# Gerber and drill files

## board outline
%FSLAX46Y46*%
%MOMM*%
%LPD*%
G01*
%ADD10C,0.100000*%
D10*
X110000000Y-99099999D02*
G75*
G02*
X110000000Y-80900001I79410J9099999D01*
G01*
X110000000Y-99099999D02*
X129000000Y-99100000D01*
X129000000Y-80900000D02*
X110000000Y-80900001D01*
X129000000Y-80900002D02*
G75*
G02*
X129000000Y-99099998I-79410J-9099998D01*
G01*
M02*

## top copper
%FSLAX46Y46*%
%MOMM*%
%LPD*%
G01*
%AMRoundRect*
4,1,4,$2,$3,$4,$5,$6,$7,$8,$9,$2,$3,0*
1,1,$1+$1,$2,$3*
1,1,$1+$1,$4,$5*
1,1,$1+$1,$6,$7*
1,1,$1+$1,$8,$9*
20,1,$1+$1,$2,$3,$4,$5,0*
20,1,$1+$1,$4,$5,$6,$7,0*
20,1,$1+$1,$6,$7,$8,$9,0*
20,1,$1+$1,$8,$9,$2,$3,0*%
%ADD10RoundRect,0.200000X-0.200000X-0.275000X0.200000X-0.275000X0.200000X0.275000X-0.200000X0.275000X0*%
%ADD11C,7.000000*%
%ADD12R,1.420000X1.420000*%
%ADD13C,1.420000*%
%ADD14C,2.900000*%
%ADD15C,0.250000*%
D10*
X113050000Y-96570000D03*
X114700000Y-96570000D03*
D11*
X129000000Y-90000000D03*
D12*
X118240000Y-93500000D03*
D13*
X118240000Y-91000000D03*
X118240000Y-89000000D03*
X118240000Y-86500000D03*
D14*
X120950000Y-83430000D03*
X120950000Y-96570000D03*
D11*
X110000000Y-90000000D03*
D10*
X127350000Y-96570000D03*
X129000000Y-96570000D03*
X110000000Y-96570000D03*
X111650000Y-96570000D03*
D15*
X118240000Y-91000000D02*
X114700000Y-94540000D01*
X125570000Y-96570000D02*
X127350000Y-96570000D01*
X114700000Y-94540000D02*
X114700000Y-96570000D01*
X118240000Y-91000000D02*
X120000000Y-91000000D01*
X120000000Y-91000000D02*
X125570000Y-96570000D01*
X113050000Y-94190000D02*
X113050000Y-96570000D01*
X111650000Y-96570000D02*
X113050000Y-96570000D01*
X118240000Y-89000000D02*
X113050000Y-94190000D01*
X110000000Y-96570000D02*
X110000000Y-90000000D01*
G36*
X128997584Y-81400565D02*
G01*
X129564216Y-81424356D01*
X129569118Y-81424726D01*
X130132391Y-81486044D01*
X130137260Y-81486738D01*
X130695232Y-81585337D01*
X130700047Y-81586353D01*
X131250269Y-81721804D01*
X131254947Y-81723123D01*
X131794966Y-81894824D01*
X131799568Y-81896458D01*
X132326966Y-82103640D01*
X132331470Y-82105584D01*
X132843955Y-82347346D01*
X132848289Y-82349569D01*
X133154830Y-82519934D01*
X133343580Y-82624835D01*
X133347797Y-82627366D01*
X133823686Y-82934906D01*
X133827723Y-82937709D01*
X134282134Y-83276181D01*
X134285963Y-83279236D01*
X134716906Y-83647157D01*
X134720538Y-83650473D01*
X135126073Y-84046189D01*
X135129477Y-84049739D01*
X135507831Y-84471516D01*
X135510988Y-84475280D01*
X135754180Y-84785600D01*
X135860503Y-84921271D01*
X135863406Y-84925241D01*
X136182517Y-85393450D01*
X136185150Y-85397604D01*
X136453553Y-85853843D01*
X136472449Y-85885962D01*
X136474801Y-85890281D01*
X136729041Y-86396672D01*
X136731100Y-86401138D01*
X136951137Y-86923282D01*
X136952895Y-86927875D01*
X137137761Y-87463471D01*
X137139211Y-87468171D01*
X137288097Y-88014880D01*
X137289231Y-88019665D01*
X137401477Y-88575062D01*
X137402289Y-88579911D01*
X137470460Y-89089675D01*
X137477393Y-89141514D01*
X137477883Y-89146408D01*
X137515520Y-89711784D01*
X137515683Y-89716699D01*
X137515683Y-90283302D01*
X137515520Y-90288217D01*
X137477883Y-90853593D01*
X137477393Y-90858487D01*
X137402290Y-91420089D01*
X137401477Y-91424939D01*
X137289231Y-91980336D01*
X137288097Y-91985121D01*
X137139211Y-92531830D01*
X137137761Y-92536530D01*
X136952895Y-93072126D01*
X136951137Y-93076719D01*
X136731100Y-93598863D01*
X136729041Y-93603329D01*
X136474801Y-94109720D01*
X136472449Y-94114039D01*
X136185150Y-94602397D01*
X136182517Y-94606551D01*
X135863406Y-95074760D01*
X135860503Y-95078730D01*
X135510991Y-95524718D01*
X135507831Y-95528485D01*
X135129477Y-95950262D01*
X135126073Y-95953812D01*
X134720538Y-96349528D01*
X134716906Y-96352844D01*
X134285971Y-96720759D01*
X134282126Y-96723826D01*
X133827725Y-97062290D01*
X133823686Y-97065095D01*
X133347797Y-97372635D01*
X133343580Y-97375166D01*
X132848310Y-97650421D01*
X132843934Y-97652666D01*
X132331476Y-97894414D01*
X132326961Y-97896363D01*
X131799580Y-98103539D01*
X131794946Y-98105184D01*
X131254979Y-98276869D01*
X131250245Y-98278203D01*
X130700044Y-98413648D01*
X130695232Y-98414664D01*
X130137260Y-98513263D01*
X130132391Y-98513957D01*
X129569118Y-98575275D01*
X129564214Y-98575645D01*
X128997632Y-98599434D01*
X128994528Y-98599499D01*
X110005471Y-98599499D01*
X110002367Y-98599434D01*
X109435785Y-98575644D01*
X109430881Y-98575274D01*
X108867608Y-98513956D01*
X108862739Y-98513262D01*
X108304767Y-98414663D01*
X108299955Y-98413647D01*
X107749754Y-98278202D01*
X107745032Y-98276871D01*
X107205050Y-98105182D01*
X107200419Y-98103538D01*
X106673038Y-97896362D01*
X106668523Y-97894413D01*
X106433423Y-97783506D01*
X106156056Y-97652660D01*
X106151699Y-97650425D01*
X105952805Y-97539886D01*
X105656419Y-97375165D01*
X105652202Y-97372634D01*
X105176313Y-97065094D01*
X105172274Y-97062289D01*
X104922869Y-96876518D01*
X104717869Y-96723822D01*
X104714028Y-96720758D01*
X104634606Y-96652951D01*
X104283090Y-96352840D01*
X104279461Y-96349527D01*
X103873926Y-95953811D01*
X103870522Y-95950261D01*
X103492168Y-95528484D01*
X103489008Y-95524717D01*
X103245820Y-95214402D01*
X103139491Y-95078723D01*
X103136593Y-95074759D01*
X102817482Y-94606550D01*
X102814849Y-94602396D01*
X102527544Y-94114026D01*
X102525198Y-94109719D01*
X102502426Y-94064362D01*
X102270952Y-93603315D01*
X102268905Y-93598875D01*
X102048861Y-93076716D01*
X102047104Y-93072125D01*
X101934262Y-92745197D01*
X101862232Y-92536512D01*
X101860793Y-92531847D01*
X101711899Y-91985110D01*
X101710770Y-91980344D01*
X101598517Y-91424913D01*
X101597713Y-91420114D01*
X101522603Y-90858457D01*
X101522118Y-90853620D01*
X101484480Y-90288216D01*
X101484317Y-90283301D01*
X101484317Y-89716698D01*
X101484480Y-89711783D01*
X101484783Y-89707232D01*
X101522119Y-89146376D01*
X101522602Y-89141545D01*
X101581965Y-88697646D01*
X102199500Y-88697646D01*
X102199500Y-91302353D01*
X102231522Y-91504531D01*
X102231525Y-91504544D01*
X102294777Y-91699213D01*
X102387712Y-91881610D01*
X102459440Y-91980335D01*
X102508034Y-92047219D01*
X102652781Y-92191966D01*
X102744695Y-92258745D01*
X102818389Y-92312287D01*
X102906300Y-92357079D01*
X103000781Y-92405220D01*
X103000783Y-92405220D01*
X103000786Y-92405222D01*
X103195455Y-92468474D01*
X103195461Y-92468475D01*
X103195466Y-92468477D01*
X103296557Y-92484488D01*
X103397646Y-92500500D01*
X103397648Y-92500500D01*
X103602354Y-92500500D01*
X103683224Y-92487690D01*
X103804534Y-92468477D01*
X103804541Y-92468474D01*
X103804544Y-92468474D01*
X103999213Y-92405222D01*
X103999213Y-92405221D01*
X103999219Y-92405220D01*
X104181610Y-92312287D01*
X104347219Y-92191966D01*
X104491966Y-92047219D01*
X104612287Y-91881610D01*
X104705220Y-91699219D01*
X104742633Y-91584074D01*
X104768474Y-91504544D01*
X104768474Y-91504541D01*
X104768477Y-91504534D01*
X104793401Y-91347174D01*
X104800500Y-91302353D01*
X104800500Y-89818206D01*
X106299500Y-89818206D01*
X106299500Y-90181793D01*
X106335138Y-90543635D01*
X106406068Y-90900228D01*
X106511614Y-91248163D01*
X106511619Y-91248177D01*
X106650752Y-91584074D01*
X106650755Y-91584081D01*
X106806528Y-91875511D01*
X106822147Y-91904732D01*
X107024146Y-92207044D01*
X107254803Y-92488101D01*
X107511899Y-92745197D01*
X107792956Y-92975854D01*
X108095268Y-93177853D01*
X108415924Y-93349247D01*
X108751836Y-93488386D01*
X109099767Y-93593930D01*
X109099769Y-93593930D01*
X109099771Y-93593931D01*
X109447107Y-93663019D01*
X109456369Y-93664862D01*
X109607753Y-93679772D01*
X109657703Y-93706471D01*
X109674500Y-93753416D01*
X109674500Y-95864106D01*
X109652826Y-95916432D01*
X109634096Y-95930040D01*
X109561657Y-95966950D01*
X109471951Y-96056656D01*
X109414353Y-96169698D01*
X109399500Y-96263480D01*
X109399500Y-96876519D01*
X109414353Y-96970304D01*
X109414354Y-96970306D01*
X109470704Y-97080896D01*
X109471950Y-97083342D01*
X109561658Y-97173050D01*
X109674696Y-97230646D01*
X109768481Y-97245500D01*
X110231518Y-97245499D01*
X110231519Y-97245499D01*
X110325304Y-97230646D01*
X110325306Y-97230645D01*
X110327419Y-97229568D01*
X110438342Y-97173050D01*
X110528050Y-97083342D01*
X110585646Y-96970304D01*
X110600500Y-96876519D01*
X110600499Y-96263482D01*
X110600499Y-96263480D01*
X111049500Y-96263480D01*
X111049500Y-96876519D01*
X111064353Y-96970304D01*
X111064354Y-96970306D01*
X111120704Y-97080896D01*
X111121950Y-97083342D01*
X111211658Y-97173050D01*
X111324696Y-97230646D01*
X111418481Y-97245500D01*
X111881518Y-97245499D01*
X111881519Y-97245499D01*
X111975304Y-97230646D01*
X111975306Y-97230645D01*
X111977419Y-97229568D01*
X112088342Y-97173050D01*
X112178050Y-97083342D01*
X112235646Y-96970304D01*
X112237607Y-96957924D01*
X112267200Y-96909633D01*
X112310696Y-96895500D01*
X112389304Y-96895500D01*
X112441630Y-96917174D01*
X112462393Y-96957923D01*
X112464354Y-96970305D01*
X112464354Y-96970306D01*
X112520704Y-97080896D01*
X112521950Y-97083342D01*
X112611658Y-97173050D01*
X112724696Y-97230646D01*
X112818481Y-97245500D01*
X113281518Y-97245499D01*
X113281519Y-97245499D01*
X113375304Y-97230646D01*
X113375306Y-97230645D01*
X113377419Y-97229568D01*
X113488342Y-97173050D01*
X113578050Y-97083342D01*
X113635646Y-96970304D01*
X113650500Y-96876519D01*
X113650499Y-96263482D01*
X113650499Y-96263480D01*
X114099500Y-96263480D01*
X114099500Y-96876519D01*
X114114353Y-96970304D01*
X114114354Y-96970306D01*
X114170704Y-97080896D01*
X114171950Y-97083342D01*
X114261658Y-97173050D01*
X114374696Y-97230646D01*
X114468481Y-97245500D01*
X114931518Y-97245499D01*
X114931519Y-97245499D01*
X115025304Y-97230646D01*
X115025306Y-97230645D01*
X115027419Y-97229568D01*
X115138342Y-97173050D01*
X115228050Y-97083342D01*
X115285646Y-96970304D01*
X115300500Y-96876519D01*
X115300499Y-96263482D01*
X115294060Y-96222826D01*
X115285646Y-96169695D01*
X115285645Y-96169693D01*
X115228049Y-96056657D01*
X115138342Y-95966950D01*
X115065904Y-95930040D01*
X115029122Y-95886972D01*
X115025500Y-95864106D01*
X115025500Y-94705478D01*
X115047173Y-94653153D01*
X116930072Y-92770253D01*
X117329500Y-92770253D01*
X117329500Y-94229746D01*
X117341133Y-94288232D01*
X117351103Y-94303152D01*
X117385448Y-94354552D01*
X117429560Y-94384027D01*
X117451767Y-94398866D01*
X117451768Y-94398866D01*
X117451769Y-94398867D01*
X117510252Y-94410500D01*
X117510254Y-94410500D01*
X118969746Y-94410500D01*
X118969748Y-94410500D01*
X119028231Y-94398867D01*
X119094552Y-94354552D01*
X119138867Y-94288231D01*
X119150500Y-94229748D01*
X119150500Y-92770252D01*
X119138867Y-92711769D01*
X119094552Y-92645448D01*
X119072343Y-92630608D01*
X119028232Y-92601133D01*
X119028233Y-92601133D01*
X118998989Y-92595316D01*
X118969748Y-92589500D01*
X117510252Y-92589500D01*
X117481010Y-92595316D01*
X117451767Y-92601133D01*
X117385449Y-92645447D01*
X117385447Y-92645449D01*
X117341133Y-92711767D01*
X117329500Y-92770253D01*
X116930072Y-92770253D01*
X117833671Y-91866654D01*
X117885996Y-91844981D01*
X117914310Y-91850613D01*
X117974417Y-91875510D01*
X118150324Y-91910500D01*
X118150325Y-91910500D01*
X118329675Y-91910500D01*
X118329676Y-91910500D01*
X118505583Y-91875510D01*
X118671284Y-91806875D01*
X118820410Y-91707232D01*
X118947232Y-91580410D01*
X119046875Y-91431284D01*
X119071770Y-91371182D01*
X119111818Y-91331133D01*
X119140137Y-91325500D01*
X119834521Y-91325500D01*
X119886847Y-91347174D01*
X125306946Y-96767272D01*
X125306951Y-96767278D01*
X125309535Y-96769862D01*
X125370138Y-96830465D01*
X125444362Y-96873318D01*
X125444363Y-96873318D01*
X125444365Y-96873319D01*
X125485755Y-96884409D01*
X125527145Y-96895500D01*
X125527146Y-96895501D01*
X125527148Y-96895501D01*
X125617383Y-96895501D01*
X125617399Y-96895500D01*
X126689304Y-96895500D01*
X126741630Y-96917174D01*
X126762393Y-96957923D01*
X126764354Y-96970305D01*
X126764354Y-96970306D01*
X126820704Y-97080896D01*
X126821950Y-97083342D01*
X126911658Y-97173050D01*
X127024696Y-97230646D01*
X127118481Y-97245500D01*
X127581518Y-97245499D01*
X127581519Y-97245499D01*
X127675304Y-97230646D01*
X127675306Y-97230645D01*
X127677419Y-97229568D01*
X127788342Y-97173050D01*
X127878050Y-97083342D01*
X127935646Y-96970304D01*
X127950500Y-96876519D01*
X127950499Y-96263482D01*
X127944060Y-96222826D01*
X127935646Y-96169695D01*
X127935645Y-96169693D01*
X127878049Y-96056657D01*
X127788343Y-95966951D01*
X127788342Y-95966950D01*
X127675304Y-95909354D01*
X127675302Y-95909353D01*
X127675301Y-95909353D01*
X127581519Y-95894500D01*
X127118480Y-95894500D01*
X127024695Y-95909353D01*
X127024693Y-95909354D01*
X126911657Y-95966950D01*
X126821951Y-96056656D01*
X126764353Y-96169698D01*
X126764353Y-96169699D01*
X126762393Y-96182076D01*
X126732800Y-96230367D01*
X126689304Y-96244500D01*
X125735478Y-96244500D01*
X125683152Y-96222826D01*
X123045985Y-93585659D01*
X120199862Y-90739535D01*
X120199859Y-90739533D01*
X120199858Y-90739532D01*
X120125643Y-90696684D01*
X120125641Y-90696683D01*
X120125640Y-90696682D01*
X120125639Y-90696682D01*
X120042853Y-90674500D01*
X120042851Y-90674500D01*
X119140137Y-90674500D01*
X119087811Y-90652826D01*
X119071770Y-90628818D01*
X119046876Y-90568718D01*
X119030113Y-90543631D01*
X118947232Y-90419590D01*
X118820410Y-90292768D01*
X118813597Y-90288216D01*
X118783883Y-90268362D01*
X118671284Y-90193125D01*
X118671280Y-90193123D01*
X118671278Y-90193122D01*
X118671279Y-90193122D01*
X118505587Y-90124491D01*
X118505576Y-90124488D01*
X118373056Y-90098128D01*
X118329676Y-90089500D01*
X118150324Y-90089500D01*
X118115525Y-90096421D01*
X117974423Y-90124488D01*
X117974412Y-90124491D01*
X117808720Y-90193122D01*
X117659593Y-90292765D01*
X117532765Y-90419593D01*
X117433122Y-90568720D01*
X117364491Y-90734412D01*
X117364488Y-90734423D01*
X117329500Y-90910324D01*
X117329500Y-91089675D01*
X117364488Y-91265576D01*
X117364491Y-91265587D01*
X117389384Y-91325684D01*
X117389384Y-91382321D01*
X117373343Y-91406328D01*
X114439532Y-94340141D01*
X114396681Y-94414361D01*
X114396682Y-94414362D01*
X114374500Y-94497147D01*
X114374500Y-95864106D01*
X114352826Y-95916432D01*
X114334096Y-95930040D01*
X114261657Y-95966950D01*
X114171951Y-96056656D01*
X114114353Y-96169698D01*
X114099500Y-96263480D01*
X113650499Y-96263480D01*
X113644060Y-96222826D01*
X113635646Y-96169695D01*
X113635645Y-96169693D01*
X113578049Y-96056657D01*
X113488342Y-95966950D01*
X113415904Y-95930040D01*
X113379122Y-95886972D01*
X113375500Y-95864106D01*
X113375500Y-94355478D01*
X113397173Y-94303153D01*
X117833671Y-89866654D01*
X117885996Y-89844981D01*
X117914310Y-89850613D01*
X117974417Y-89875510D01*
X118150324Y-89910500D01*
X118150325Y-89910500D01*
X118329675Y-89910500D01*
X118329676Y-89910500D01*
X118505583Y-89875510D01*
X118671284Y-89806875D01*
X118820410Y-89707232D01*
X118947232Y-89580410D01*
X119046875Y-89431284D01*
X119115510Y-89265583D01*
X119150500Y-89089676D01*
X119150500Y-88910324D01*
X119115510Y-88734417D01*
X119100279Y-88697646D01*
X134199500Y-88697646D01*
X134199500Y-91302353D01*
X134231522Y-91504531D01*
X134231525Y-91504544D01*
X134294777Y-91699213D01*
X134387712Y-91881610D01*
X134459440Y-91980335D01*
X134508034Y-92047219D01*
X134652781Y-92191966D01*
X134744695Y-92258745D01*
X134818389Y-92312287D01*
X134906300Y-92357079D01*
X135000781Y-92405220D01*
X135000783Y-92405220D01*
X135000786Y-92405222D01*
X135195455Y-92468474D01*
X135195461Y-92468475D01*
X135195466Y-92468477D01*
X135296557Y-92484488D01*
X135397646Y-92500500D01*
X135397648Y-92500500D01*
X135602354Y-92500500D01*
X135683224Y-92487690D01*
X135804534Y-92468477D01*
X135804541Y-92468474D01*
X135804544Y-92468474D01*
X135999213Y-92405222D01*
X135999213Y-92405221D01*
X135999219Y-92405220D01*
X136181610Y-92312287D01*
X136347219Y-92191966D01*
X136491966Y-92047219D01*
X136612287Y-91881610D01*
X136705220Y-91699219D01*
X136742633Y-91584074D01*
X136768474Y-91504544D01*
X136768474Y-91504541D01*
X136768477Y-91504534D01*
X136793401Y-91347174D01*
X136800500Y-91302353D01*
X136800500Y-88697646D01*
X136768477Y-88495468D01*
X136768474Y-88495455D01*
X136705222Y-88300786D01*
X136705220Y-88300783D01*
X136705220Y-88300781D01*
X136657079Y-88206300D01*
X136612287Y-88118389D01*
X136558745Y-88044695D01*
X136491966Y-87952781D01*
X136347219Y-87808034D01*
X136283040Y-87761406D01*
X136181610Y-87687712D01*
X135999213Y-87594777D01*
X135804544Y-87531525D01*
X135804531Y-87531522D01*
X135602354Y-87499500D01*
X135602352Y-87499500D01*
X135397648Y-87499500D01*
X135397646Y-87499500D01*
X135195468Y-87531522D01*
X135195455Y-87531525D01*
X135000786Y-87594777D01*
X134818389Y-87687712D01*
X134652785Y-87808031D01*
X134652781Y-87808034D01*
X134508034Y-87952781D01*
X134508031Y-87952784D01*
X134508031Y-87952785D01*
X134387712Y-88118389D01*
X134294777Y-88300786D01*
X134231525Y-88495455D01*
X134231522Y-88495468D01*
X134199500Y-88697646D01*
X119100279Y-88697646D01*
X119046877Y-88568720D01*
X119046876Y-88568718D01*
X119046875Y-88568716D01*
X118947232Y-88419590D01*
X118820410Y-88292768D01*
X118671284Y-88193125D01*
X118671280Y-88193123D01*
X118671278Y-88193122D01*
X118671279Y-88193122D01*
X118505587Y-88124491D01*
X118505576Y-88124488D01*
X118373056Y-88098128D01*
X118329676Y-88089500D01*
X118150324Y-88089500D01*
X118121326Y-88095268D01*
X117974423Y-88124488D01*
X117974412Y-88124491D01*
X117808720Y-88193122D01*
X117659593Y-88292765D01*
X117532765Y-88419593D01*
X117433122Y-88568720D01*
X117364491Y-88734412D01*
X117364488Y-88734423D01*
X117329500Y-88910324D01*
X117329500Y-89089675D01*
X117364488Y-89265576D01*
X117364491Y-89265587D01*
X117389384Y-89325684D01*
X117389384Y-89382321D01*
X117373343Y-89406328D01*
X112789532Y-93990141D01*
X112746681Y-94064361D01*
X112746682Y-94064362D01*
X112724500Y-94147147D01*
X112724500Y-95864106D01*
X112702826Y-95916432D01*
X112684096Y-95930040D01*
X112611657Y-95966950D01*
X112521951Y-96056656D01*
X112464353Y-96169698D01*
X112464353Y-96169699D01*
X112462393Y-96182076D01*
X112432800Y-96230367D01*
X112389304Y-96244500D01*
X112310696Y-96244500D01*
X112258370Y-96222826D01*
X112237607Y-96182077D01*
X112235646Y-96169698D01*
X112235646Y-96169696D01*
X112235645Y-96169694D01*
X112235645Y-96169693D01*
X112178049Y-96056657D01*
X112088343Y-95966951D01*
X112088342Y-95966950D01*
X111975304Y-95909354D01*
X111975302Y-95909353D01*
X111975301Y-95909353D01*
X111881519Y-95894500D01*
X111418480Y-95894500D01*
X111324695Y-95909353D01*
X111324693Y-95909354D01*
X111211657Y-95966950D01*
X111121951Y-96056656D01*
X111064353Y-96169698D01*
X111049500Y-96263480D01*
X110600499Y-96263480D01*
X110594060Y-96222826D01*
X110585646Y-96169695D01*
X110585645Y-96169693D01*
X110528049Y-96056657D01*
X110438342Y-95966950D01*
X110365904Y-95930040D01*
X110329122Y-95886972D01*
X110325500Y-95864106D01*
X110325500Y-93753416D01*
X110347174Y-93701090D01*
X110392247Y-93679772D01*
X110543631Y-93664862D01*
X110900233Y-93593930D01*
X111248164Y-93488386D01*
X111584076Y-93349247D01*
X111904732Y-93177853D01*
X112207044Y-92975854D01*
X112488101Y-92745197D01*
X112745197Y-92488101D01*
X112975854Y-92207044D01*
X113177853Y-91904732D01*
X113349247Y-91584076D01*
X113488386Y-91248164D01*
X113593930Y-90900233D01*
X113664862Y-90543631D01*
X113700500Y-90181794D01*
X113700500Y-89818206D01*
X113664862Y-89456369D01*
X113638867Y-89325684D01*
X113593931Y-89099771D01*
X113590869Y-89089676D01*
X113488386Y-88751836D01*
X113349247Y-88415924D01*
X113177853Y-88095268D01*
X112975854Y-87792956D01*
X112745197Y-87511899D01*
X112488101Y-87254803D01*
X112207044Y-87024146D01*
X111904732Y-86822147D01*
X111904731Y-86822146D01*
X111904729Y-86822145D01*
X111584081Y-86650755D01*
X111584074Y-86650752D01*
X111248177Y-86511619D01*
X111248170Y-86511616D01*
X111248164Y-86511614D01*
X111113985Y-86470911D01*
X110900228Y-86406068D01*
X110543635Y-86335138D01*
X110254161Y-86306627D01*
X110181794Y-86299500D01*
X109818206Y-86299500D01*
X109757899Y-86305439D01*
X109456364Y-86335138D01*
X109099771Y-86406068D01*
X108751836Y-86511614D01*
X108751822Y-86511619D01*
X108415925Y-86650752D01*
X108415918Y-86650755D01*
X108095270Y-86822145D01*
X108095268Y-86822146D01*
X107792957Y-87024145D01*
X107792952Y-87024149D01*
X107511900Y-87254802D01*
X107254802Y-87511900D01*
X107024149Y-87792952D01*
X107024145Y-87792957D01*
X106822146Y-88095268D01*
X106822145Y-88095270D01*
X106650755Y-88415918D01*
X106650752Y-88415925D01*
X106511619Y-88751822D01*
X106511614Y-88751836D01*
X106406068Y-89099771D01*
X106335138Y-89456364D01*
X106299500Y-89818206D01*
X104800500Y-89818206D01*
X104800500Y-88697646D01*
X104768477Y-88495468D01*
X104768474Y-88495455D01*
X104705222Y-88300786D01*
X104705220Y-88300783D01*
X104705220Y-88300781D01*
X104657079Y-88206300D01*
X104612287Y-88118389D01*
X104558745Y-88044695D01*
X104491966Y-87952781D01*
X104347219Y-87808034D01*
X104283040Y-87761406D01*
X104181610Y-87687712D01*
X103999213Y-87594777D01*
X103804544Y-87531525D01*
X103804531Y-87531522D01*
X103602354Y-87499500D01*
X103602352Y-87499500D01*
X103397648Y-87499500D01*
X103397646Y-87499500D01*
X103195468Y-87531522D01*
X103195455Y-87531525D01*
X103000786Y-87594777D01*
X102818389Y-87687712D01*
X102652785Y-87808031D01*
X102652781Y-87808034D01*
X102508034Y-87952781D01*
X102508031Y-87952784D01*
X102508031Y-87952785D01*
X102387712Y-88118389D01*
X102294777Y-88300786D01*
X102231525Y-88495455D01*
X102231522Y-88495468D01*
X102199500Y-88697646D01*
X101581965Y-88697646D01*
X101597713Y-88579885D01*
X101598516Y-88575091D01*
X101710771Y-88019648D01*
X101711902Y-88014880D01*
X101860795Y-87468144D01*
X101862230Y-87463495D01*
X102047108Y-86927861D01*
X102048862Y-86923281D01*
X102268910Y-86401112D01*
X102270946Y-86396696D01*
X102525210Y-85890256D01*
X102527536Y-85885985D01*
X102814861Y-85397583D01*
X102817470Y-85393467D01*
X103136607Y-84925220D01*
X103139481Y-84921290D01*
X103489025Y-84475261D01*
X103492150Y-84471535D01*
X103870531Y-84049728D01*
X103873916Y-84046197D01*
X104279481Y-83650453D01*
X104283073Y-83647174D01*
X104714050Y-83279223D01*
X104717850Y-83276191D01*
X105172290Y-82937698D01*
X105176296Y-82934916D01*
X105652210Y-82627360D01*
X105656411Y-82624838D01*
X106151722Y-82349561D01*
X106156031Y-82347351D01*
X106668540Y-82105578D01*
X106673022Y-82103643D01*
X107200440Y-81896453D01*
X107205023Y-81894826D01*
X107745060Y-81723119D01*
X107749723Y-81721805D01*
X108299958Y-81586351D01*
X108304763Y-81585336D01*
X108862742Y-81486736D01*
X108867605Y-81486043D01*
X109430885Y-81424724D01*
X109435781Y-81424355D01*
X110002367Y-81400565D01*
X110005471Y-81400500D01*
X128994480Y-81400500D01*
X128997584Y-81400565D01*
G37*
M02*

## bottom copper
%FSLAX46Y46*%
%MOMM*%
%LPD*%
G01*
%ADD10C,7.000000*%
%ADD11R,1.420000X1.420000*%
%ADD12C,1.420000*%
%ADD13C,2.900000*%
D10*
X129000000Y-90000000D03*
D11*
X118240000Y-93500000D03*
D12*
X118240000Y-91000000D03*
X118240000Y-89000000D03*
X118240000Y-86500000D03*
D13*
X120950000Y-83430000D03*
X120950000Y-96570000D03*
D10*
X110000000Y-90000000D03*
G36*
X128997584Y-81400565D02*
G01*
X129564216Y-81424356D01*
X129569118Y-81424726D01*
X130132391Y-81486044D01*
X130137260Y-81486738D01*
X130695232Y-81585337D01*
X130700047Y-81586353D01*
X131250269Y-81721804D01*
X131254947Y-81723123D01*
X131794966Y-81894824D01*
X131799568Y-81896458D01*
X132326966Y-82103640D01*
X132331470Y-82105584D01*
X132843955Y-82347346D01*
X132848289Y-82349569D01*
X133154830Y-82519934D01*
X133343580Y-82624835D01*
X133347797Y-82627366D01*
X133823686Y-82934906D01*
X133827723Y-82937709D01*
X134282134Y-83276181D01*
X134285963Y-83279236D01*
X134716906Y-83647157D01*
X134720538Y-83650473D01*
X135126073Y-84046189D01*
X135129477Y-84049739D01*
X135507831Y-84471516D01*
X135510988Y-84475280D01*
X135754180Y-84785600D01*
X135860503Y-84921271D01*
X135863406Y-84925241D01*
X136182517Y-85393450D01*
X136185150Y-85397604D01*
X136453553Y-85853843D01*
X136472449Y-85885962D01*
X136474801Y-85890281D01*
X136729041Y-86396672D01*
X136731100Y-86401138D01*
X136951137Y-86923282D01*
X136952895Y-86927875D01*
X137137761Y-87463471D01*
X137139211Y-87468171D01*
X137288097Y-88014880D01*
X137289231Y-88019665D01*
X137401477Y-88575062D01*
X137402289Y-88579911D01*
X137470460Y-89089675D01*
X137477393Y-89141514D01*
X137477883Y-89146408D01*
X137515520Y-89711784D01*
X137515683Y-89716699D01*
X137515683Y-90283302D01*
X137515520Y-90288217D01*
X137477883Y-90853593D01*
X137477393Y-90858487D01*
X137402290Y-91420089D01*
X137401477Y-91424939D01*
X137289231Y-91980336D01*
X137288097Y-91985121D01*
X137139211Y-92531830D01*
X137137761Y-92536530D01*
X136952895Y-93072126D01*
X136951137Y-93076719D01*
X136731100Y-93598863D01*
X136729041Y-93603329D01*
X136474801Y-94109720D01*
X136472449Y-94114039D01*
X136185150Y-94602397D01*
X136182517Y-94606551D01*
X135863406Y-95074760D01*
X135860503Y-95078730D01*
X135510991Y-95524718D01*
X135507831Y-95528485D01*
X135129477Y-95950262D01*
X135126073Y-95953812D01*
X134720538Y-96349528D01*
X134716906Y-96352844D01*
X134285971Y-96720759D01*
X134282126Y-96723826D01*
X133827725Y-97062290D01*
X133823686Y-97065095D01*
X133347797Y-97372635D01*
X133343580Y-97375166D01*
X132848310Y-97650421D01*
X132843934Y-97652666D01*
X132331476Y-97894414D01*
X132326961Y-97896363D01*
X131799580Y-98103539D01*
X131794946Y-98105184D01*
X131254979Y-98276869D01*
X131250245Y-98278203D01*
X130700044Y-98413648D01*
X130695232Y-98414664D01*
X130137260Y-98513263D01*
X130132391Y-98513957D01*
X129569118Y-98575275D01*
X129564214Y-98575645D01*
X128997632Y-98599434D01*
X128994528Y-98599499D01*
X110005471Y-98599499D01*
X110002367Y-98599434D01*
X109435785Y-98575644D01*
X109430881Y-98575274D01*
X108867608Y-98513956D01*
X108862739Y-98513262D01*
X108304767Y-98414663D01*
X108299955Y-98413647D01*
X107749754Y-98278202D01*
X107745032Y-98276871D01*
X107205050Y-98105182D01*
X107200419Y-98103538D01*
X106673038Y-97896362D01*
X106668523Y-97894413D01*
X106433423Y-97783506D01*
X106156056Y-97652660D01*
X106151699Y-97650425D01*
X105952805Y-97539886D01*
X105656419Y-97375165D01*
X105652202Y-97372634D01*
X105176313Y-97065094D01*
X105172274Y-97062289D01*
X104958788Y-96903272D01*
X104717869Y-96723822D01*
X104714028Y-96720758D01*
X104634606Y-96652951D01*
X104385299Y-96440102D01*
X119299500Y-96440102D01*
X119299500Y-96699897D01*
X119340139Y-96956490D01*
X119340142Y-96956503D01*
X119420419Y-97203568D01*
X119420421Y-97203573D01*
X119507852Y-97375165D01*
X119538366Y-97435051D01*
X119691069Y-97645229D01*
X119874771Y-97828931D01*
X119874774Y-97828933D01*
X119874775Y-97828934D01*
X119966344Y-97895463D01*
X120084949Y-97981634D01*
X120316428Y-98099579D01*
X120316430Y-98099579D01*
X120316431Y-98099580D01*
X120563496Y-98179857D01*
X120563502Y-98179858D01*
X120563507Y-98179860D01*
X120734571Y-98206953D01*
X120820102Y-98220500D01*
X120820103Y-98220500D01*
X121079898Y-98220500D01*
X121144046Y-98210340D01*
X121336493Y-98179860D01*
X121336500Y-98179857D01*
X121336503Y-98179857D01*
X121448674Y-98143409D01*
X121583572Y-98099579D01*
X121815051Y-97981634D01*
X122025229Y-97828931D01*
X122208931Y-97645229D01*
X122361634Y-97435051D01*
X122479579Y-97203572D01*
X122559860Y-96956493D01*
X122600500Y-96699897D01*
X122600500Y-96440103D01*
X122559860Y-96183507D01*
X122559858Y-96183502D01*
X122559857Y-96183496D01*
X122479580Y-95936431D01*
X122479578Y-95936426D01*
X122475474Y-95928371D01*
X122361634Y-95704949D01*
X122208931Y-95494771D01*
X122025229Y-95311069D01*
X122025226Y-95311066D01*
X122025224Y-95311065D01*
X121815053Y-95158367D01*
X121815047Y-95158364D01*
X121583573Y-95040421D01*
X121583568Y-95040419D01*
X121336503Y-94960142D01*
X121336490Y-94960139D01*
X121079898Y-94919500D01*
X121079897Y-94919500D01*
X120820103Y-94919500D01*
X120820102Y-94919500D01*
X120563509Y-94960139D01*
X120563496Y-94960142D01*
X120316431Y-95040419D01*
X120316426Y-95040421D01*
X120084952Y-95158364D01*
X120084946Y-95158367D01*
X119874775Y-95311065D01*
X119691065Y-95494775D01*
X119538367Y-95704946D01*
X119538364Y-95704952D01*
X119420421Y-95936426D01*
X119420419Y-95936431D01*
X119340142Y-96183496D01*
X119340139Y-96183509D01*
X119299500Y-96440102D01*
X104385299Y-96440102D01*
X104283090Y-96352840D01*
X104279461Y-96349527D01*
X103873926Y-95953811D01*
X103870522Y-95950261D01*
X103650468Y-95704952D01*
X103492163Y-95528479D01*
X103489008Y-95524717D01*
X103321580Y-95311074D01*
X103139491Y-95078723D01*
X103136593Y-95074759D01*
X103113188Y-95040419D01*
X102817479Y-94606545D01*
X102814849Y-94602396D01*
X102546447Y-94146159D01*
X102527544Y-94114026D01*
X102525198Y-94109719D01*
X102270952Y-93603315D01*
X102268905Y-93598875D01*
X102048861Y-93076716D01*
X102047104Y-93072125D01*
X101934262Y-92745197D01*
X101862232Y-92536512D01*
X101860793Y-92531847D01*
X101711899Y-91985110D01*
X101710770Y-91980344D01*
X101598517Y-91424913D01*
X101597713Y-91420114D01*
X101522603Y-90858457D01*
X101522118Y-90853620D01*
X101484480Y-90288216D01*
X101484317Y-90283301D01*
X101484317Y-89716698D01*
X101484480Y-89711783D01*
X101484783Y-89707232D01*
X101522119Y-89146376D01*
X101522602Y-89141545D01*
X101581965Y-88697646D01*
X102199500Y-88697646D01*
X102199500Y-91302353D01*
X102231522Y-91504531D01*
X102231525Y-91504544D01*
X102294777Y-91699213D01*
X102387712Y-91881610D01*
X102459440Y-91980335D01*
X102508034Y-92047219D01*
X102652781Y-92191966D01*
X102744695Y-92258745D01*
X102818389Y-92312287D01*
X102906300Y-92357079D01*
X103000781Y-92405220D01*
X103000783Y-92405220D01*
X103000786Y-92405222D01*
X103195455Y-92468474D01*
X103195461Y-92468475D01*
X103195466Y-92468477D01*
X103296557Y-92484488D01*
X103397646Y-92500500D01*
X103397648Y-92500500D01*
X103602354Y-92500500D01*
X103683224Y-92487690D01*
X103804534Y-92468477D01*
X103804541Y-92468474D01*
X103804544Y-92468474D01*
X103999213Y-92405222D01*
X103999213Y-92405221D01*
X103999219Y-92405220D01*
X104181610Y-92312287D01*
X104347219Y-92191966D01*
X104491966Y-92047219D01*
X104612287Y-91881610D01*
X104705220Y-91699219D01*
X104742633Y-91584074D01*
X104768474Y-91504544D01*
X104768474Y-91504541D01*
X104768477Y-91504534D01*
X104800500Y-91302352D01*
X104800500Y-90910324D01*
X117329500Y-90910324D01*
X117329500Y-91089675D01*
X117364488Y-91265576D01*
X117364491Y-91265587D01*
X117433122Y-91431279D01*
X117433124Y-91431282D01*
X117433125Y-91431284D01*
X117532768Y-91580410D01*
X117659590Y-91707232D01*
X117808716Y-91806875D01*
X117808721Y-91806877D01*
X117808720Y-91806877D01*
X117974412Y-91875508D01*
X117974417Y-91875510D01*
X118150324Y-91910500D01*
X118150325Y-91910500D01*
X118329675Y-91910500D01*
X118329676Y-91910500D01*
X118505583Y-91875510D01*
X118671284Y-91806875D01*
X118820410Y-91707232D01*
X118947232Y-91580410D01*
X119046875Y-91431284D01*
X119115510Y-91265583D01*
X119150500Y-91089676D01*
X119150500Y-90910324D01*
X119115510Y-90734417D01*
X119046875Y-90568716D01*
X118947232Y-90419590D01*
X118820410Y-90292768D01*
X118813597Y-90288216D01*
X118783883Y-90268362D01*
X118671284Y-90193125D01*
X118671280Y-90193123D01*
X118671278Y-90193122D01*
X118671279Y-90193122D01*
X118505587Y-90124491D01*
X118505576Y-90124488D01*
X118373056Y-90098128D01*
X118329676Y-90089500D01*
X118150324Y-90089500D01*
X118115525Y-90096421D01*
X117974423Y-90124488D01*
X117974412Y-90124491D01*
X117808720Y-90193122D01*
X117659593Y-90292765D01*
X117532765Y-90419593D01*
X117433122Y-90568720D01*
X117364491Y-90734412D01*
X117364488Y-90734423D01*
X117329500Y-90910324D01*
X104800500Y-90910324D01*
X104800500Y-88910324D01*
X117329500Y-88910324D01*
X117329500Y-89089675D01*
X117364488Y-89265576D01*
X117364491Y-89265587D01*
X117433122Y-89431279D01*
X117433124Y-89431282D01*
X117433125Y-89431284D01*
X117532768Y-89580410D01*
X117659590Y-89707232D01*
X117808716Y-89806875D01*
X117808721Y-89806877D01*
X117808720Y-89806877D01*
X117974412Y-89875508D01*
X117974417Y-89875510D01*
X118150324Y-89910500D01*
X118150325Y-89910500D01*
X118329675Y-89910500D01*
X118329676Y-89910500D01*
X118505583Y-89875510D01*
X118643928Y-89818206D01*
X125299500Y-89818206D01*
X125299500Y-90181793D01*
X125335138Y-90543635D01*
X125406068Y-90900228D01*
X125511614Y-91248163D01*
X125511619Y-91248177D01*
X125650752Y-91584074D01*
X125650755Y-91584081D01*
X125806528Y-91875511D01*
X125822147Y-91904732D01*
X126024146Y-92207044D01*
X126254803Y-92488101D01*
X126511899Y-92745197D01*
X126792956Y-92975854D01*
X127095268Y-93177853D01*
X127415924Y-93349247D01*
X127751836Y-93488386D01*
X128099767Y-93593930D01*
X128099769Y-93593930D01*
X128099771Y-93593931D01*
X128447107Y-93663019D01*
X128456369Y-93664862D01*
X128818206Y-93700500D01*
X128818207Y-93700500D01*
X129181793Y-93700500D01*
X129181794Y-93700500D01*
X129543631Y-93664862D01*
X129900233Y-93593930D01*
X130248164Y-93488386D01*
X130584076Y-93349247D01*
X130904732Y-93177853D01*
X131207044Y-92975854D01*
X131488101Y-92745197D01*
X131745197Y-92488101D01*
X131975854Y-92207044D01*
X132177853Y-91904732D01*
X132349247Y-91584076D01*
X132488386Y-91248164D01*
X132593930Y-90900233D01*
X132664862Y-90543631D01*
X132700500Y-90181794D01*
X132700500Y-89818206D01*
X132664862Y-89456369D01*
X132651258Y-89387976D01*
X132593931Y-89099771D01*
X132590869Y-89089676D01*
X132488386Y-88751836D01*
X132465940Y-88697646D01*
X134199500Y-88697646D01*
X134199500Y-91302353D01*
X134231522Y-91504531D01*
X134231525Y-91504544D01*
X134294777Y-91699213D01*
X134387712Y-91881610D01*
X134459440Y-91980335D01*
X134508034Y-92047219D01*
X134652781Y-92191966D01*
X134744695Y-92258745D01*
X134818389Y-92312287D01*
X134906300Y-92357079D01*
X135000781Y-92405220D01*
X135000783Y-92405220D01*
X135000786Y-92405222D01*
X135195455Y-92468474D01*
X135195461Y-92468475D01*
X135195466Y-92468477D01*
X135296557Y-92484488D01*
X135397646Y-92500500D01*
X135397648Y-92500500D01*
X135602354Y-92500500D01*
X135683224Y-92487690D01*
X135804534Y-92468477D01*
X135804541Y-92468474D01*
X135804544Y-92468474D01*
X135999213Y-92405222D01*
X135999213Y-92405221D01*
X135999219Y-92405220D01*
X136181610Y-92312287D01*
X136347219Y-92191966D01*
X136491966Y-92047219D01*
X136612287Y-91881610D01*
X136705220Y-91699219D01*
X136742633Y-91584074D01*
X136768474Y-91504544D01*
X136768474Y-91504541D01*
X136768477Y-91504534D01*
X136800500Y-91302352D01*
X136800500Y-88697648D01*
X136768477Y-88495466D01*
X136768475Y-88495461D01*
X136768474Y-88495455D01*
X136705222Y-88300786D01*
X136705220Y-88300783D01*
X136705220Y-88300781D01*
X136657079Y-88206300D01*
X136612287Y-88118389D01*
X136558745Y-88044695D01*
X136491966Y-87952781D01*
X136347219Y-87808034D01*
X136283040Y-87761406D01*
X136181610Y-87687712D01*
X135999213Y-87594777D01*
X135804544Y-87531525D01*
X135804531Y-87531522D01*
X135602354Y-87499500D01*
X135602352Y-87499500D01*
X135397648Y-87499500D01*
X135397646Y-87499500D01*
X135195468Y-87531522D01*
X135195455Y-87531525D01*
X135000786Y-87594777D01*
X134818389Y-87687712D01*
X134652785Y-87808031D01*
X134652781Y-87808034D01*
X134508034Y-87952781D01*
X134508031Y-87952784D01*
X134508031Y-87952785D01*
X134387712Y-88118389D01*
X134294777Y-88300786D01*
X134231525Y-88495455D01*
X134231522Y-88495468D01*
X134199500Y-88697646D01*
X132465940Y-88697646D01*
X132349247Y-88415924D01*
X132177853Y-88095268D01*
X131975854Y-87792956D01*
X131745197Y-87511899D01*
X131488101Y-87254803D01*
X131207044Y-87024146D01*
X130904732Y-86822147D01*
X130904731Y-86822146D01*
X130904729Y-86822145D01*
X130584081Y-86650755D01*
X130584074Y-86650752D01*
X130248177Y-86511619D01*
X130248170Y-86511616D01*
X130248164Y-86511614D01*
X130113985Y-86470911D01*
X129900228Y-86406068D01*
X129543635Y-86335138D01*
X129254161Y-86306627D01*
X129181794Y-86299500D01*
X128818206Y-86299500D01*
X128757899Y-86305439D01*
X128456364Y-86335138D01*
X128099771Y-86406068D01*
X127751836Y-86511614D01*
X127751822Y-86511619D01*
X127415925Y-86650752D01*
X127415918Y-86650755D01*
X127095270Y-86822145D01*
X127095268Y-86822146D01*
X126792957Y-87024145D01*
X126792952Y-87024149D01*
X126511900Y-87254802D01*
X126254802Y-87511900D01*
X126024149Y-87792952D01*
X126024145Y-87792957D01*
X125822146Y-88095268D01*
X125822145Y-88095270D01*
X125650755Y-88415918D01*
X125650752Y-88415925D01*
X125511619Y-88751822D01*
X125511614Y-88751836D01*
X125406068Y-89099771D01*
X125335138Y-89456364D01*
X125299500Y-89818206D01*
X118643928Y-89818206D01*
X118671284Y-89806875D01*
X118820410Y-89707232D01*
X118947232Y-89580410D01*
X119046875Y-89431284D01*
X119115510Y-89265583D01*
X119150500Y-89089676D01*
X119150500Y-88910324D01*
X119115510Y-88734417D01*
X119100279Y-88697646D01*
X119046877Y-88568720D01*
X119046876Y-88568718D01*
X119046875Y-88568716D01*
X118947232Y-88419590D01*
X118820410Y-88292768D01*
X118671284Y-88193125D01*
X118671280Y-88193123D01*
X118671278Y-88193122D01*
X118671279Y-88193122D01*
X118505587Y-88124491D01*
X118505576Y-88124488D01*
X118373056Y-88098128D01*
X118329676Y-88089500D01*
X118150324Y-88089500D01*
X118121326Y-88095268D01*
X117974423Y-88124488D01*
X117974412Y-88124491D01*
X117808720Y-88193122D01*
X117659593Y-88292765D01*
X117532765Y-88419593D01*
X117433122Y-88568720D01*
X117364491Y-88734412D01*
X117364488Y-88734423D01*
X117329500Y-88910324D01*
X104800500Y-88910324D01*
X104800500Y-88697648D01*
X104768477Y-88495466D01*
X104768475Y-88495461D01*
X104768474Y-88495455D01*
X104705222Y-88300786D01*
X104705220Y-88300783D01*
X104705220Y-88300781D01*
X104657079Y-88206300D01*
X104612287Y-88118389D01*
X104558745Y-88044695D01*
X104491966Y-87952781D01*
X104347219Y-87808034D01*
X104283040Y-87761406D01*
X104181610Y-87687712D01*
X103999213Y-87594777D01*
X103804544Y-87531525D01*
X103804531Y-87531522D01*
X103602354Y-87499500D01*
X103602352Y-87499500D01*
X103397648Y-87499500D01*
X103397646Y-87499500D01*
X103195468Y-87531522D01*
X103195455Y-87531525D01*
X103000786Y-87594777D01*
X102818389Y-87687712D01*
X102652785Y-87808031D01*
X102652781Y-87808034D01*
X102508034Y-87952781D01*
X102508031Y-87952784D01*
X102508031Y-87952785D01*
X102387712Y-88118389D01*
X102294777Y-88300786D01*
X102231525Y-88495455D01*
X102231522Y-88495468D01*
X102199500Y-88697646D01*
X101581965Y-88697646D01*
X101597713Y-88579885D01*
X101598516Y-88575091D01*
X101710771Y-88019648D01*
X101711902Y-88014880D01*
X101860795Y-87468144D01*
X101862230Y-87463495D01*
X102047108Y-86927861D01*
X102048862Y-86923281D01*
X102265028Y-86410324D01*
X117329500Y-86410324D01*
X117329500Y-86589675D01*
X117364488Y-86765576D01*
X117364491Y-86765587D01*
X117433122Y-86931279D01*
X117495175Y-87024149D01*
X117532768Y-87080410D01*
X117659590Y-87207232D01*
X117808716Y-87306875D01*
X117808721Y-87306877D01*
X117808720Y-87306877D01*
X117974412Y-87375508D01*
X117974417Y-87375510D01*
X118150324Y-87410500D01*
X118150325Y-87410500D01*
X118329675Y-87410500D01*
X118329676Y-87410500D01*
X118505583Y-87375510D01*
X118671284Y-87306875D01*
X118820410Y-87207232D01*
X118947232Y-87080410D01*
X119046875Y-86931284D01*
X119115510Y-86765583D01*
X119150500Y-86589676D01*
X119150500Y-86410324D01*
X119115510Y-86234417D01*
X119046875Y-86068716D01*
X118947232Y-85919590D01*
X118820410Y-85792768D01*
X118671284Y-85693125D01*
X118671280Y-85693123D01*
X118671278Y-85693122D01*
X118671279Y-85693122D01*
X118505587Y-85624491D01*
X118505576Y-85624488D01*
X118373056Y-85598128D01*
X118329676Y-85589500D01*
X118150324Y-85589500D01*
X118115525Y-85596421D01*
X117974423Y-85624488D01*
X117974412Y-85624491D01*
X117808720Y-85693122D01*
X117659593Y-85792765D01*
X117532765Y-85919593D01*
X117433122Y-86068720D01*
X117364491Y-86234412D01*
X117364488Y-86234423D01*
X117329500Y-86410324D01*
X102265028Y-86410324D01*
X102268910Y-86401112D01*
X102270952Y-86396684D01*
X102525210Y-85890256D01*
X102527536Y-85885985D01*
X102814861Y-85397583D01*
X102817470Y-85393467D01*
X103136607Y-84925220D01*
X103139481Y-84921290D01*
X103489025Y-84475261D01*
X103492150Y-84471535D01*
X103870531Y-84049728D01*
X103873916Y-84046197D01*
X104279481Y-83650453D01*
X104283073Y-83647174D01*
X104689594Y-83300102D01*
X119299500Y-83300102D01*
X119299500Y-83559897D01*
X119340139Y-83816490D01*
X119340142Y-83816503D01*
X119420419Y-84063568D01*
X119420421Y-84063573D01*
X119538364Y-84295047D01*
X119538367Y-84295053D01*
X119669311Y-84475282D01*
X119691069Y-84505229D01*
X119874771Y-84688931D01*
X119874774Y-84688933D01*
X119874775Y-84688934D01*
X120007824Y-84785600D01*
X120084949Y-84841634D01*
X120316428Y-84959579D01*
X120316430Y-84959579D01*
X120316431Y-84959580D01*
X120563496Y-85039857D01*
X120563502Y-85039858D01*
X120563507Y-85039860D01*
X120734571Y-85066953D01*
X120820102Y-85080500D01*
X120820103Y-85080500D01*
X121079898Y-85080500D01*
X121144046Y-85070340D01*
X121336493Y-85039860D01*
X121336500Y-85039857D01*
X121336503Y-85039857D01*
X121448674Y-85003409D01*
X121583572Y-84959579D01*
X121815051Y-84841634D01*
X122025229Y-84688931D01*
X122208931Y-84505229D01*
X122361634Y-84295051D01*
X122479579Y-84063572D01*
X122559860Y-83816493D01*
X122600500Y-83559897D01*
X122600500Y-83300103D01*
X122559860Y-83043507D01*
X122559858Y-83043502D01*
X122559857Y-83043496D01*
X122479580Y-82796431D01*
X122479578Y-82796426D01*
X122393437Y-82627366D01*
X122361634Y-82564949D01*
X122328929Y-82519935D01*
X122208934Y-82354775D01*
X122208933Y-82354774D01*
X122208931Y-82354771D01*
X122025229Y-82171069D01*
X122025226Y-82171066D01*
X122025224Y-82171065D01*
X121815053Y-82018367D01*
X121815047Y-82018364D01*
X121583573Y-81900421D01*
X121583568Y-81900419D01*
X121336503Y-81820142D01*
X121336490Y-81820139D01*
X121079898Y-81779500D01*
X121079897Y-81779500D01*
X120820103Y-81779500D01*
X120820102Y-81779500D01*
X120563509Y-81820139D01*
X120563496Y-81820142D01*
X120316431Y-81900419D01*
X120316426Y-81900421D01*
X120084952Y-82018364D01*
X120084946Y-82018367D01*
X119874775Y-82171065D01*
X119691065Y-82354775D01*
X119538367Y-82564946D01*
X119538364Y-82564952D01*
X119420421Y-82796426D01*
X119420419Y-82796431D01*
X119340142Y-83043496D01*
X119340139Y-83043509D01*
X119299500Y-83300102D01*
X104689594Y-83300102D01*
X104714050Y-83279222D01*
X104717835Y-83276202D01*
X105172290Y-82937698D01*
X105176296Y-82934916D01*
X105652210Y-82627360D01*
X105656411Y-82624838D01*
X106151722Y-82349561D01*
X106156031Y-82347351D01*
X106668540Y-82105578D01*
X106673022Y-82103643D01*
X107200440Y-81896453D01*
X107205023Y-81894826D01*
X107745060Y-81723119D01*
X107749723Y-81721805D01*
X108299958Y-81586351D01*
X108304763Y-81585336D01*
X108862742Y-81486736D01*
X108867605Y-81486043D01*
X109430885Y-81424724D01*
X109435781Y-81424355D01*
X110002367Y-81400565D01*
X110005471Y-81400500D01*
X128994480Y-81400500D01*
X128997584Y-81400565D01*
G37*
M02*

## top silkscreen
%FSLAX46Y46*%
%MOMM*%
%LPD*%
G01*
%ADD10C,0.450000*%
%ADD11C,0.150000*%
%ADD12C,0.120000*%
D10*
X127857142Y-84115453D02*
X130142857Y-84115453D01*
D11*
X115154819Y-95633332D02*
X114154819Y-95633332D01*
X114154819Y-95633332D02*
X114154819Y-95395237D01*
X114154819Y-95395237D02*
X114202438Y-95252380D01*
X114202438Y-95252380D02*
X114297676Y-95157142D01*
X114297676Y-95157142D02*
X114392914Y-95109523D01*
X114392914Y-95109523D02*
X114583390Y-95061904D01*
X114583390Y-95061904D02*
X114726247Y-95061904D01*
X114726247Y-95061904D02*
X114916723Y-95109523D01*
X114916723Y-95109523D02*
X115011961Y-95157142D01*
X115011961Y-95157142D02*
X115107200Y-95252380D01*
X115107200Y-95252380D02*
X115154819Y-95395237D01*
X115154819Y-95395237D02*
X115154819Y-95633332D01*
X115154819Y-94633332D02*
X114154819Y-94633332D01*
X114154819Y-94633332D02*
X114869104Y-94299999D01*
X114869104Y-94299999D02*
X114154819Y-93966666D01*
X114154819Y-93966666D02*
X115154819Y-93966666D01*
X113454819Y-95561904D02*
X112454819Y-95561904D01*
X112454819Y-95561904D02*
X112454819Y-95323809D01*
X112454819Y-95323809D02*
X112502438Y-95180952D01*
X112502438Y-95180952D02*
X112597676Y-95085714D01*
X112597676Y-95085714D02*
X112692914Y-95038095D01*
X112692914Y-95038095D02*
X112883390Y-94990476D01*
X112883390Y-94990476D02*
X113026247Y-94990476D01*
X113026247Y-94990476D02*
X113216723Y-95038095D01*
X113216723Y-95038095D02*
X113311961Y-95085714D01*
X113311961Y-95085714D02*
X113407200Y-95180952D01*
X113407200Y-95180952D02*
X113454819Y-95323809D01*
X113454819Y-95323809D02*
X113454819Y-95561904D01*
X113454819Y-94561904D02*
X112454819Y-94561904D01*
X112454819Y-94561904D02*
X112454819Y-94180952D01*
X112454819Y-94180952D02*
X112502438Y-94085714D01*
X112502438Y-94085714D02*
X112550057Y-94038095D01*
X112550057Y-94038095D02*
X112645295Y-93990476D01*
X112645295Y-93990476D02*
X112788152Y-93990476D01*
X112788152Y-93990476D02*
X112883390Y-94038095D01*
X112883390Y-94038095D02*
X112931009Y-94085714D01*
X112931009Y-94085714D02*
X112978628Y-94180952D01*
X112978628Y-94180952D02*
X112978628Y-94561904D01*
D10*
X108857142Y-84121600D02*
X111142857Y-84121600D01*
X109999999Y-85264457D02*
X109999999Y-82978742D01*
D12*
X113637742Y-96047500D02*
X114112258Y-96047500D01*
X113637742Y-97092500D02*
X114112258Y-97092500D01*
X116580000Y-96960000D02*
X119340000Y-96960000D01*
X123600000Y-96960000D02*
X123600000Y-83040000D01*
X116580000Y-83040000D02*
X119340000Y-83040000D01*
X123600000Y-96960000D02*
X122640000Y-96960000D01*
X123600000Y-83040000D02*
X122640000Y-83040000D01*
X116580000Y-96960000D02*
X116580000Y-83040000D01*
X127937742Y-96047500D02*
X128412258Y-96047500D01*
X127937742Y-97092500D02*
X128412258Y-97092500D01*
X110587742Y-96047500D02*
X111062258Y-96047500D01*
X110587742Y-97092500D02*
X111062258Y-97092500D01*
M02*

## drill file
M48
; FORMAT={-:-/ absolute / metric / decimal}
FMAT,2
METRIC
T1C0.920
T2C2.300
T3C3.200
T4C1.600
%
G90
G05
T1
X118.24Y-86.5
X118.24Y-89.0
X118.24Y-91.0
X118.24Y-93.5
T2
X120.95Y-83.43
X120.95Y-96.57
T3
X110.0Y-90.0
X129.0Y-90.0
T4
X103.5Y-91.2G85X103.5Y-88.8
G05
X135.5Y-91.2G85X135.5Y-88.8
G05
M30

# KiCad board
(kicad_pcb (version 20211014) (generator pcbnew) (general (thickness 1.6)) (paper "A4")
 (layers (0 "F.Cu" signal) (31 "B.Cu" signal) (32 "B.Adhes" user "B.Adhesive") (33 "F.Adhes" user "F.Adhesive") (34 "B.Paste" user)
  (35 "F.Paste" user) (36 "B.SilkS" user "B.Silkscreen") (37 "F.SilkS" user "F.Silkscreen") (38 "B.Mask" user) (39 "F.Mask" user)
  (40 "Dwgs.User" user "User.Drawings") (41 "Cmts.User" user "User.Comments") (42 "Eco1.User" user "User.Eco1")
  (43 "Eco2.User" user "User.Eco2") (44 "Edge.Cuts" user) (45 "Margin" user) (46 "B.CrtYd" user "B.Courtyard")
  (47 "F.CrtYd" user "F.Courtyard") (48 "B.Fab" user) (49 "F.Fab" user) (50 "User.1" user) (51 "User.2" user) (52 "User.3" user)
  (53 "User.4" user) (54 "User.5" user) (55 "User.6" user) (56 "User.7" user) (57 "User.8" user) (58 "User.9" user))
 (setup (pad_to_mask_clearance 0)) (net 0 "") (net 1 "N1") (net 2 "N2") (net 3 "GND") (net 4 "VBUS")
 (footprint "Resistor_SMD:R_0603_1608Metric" (layer "F.Cu") (at 113.875 96.57)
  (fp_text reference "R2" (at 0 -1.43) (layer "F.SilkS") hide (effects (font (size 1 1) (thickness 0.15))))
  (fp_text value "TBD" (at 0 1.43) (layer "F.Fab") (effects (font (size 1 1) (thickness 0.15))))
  (fp_line (start -0.237258 -0.5225) (end 0.237258 -0.5225) (layer "F.SilkS") (width 0.12))
  (fp_line (start -0.237258 0.5225) (end 0.237258 0.5225) (layer "F.SilkS") (width 0.12))
  (pad "1" smd roundrect locked (at -0.825 0) (size 0.8 0.95) (layers "F.Cu" "F.Paste" "F.Mask") (roundrect_rratio 0.25) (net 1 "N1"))
  (pad "2" smd roundrect locked (at 0.825 0) (size 0.8 0.95) (layers "F.Cu" "F.Paste" "F.Mask") (roundrect_rratio 0.25) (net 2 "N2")))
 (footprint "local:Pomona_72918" (layer "F.Cu") (at 129 90)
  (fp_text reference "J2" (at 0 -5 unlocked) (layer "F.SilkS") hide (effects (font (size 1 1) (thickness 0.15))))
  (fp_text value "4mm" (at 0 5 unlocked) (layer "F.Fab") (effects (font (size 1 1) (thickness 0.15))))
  (pad "1" thru_hole circle (at 0 0) (size 7 7) (drill 3.2) (layers *.Cu *.Mask) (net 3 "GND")))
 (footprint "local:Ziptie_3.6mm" (layer "F.Cu") (at 135.5 90 90)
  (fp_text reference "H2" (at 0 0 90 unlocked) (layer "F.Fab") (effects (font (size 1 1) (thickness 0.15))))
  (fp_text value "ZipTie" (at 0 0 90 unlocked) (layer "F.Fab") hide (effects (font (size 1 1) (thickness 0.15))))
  (pad "" np_thru_hole oval (at 0 0 90) (size 4 1.6) (drill oval 4 1.6) (layers F&B.Cu *.Mask)))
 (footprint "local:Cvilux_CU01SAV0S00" (layer "F.Cu") (at 118.24 93.5 90)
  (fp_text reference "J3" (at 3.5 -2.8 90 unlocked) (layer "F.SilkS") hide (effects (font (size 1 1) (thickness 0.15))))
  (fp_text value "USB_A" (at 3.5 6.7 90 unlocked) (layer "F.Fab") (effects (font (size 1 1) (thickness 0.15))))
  (fp_line (start -3.46 -1.66) (end -3.46 1.1) (layer "F.SilkS") (width 0.12))
  (fp_line (start -3.46 5.36) (end 10.46 5.36) (layer "F.SilkS") (width 0.12))
  (fp_line (start 10.46 -1.66) (end 10.46 1.1) (layer "F.SilkS") (width 0.12))
  (fp_line (start -3.46 5.36) (end -3.46 4.4) (layer "F.SilkS") (width 0.12))
  (fp_line (start 10.46 5.36) (end 10.46 4.4) (layer "F.SilkS") (width 0.12))
  (fp_line (start -3.46 -1.66) (end 10.46 -1.66) (layer "F.SilkS") (width 0.12))
  (pad "1" thru_hole rect (at 0 0 90) (size 1.42 1.42) (drill 0.92) (layers *.Cu *.Mask) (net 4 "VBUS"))
  (pad "2" thru_hole circle (at 2.5 0 90) (size 1.42 1.42) (drill 0.92) (layers *.Cu *.Mask) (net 2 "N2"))
  (pad "3" thru_hole circle (at 4.5 0 90) (size 1.42 1.42) (drill 0.92) (layers *.Cu *.Mask) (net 1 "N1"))
  (pad "4" thru_hole circle (at 7 0 90) (size 1.42 1.42) (drill 0.92) (layers *.Cu *.Mask) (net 3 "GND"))
  (pad "5" thru_hole circle (at 10.07 2.71 90) (size 2.9 2.9) (drill 2.3) (layers *.Cu *.Mask) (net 3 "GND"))
  (pad "5" thru_hole circle (at -3.07 2.71 90) (size 2.9 2.9) (drill 2.3) (layers *.Cu *.Mask) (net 3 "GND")))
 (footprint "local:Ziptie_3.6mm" (layer "F.Cu") (at 103.5 90 90)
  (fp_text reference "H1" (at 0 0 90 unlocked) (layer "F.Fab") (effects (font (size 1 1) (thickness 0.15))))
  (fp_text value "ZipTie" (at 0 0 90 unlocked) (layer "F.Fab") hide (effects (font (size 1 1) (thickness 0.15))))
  (pad "" np_thru_hole oval (at 0 0 90) (size 4 1.6) (drill oval 4 1.6) (layers F&B.Cu *.Mask)))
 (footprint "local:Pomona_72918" (layer "F.Cu") (at 110 90)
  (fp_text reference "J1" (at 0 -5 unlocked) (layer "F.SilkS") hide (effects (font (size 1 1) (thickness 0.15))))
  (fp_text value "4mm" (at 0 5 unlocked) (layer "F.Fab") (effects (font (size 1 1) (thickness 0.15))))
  (pad "1" thru_hole circle (at 0 0) (size 7 7) (drill 3.2) (layers *.Cu *.Mask) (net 4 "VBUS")))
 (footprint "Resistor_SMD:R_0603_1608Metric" (layer "F.Cu") (at 128.175 96.57)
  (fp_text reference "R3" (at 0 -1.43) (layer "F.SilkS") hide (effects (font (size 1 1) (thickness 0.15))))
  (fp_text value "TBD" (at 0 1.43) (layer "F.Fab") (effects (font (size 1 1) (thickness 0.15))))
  (fp_line (start -0.237258 -0.5225) (end 0.237258 -0.5225) (layer "F.SilkS") (width 0.12))
  (fp_line (start -0.237258 0.5225) (end 0.237258 0.5225) (layer "F.SilkS") (width 0.12))
  (pad "1" smd roundrect locked (at -0.825 0) (size 0.8 0.95) (layers "F.Cu" "F.Paste" "F.Mask") (roundrect_rratio 0.25) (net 2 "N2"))
  (pad "2" smd roundrect locked (at 0.825 0) (size 0.8 0.95) (layers "F.Cu" "F.Paste" "F.Mask") (roundrect_rratio 0.25) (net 3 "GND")))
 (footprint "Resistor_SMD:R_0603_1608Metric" (layer "F.Cu") (at 110.825 96.57)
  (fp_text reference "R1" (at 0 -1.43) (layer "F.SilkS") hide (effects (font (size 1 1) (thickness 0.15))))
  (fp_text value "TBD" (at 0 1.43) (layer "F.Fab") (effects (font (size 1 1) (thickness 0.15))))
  (fp_line (start -0.237258 -0.5225) (end 0.237258 -0.5225) (layer "F.SilkS") (width 0.12))
  (fp_line (start -0.237258 0.5225) (end 0.237258 0.5225) (layer "F.SilkS") (width 0.12))
  (pad "1" smd roundrect locked (at -0.825 0) (size 0.8 0.95) (layers "F.Cu" "F.Paste" "F.Mask") (roundrect_rratio 0.25) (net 4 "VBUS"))
  (pad "2" smd roundrect locked (at 0.825 0) (size 0.8 0.95) (layers "F.Cu" "F.Paste" "F.Mask") (roundrect_rratio 0.25) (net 1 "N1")))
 (gr_arc (start 110 99.099999) (mid 100.979068 90) (end 110 80.900001) (layer "Edge.Cuts") (width 0.1))
 (gr_line (start 110 99.099999) (end 129 99.1) (layer "Edge.Cuts") (width 0.1))
 (gr_line (start 129 80.9) (end 110 80.900001) (layer "Edge.Cuts") (width 0.1))
 (gr_arc (start 129 80.900002) (mid 138.020932 90.000001) (end 129 99.1) (layer "Edge.Cuts") (width 0.1))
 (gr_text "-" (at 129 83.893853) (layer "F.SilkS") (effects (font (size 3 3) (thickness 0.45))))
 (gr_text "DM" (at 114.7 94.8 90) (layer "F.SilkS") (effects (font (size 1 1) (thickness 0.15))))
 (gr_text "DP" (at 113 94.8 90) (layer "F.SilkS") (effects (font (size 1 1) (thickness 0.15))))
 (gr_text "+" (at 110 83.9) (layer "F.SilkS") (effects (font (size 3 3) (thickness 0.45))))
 (segment (start 118.24 91) (end 114.7 94.54) (width 0.25) (layer "F.Cu") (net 2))
 (segment (start 125.57 96.57) (end 127.35 96.57) (width 0.25) (layer "F.Cu") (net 2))
 (segment (start 114.7 94.54) (end 114.7 96.57) (width 0.25) (layer "F.Cu") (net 2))
 (segment (start 118.24 91) (end 120 91) (width 0.25) (layer "F.Cu") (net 2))
 (segment (start 120 91) (end 125.57 96.57) (width 0.25) (layer "F.Cu") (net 2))
 (segment (start 113.05 94.19) (end 113.05 96.57) (width 0.25) (layer "F.Cu") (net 1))
 (segment (start 111.65 96.57) (end 113.05 96.57) (width 0.25) (layer "F.Cu") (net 1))
 (segment (start 118.24 89) (end 113.05 94.19) (width 0.25) (layer "F.Cu") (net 1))
 (segment (start 110 96.57) (end 110 90) (width 0.25) (layer "F.Cu") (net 4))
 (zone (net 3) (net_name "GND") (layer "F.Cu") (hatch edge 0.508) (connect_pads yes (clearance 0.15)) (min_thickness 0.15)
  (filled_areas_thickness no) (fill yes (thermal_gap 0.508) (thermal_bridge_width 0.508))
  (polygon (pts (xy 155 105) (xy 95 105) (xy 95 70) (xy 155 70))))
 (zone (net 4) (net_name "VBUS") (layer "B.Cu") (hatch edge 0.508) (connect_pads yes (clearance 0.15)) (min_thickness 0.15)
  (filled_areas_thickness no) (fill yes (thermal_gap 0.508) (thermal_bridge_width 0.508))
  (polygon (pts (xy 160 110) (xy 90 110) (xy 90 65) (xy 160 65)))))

